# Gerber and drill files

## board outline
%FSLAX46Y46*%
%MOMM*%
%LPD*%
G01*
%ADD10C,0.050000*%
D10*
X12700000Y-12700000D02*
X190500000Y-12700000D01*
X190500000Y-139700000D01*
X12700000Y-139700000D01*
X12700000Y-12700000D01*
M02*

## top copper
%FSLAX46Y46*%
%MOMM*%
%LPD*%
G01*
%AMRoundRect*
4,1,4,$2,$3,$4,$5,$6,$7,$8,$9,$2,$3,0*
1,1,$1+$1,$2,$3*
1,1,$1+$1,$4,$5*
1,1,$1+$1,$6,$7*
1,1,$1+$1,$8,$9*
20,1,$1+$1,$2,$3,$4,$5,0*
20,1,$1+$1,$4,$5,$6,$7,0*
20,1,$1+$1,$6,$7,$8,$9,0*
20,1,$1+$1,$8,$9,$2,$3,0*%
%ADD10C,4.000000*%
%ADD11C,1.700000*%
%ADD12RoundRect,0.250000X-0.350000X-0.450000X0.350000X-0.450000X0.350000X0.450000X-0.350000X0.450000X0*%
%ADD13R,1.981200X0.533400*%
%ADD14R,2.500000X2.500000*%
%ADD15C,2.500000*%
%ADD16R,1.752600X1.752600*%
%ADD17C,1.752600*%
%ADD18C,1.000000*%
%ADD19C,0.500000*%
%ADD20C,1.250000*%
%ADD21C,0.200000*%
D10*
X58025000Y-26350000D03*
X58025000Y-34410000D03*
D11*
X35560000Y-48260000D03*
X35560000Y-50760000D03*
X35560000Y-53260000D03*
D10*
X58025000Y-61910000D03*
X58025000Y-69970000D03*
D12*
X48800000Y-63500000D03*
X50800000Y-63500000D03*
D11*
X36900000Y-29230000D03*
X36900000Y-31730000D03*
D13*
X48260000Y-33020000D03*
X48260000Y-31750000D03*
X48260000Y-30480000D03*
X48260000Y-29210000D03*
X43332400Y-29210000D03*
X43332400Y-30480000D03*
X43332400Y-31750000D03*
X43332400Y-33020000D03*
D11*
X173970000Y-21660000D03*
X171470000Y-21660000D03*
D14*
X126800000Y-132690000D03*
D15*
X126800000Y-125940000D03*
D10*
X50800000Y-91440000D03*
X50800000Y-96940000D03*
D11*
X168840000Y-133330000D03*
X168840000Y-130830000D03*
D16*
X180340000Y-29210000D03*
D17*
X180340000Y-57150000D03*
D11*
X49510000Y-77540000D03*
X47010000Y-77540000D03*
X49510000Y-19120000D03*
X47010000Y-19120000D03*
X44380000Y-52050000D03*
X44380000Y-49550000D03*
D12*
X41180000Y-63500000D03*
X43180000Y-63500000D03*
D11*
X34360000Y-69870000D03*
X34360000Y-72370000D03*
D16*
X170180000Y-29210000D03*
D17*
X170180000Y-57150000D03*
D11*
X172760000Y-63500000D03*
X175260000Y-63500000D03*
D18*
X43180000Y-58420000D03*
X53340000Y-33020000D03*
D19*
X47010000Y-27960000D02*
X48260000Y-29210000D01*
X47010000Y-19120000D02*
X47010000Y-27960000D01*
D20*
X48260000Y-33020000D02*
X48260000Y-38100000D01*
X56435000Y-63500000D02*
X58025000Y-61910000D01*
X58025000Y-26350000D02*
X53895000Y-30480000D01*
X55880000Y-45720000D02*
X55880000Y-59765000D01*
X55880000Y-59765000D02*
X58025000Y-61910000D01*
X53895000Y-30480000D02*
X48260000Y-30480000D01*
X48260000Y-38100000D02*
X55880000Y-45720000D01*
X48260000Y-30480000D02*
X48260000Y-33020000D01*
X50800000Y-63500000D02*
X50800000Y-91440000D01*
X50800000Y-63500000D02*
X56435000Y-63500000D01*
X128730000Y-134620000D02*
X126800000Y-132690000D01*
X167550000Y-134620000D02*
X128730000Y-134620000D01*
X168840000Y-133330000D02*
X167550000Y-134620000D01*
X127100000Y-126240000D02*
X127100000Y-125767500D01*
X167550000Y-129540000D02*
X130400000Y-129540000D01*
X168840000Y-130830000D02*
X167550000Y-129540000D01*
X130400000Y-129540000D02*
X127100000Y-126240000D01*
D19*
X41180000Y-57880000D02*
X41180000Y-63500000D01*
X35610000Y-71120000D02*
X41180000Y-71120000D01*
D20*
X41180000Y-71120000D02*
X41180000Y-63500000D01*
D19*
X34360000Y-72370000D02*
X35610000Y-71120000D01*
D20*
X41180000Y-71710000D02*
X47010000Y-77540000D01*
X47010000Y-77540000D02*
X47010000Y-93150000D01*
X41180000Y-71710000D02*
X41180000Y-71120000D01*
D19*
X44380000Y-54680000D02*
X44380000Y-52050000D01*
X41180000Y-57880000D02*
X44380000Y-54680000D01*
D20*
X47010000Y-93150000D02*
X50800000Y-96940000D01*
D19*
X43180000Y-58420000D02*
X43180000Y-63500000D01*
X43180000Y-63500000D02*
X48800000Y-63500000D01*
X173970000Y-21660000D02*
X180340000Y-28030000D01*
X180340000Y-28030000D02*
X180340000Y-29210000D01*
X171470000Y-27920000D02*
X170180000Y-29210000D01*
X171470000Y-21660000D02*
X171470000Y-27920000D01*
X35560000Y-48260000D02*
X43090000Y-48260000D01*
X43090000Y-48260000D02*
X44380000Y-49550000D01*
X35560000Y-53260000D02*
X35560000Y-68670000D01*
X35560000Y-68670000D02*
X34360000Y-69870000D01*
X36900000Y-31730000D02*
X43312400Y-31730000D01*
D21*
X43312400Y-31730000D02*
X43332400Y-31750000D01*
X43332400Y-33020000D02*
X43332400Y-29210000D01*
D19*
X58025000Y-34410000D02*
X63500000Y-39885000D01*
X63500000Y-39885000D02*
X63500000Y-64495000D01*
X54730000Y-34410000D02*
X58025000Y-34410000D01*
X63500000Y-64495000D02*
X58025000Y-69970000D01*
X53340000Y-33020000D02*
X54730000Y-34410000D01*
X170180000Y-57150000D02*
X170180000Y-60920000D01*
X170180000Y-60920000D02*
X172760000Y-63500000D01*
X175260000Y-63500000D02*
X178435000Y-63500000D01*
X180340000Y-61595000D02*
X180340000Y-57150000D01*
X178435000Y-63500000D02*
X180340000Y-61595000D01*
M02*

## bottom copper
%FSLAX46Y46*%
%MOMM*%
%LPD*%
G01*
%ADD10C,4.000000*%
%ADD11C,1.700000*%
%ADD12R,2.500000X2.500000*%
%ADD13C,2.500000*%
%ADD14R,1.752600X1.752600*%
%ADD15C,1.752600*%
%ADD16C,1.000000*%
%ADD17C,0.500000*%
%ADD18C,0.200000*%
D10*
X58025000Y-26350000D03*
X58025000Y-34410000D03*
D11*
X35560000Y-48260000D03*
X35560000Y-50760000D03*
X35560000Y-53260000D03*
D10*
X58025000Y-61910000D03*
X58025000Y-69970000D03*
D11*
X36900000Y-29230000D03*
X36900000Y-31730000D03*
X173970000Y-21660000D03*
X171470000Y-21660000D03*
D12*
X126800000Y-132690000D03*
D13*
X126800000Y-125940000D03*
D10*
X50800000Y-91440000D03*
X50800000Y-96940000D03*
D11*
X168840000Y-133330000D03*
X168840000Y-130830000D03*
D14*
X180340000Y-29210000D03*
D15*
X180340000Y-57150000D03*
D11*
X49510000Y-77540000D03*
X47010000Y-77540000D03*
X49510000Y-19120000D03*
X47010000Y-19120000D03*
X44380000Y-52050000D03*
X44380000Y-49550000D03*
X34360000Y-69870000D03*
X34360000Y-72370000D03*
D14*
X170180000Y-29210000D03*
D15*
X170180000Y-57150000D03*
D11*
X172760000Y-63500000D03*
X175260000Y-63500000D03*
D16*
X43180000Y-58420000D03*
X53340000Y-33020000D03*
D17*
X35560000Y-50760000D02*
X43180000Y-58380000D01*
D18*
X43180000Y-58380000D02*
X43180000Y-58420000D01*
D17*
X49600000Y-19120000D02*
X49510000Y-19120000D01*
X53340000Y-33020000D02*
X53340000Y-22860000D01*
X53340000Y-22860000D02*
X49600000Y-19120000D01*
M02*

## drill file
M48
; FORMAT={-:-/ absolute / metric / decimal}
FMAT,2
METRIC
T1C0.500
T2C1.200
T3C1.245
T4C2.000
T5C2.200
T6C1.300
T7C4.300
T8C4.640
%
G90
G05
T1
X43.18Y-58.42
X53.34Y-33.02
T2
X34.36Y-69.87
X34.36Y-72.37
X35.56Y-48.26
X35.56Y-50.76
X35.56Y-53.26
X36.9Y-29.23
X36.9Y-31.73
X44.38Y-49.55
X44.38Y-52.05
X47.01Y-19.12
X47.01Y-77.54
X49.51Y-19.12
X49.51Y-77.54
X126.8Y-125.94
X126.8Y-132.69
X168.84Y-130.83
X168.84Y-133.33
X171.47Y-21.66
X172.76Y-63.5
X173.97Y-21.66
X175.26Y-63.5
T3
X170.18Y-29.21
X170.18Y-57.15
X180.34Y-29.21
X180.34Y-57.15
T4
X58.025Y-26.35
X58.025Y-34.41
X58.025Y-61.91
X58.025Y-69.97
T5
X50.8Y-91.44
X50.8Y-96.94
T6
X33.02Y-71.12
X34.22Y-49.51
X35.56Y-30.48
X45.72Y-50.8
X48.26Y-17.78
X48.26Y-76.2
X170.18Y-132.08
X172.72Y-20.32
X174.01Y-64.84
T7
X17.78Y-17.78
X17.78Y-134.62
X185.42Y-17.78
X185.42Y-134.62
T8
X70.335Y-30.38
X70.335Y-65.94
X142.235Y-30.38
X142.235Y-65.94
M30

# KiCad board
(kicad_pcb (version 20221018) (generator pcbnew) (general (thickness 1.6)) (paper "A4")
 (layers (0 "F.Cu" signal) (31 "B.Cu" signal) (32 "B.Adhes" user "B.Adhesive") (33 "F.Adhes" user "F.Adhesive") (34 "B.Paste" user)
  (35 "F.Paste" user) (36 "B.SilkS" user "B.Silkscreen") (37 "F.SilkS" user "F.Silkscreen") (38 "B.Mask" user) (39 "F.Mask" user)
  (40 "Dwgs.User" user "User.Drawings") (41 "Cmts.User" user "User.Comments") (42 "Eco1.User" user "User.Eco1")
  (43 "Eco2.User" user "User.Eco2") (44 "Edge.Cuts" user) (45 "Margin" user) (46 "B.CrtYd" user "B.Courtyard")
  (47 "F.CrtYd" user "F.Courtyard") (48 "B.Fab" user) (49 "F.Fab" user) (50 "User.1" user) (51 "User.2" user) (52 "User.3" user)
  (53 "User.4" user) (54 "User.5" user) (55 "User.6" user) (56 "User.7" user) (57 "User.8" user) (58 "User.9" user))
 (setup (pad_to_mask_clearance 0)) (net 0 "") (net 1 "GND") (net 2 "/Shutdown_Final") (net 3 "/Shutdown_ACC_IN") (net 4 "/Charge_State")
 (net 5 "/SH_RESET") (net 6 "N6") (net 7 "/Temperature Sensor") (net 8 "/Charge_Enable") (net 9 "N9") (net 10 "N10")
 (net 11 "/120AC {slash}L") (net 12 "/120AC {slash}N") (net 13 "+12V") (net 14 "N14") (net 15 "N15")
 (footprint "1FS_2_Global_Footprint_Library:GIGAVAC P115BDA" (layer "F.Cu") (at 146.925 46.95 180)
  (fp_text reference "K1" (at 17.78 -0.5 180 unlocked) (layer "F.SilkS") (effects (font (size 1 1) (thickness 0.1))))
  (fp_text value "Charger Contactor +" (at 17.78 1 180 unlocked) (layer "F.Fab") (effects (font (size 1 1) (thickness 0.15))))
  (pad "" np_thru_hole circle (at 4.69 16.57 180) (size 4.64 4.64) (drill 4.64) (layers "F&B.Cu" "*.Mask"))
  (pad "" np_thru_hole circle (at 76.59 16.57 180) (size 4.64 4.64) (drill 4.64) (layers "F&B.Cu" "*.Mask"))
  (pad "3" thru_hole circle (at 88.9 20.6 180) (size 4 4) (drill 2) (layers "*.Cu" "*.Mask") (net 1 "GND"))
  (pad "4" thru_hole circle (at 88.9 12.54 180) (size 4 4) (drill 2) (layers "*.Cu" "*.Mask") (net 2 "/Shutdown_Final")))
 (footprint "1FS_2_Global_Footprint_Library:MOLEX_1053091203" (layer "F.Cu") (at 35.56 48.26 -90)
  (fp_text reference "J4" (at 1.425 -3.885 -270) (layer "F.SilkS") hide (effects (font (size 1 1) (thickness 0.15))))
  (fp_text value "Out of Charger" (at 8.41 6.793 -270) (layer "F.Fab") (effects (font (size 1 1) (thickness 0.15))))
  (pad "" np_thru_hole circle (at 1.25 1.34 270) (size 1.3 1.3) (drill 1.3) (layers "*.Cu" "*.Mask"))
  (pad "1" thru_hole circle (at 0 0 270) (size 1.7 1.7) (drill 1.2) (layers "*.Cu") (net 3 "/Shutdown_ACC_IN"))
  (pad "2" thru_hole circle (at 2.5 0 270) (size 1.7 1.7) (drill 1.2) (layers "*.Cu") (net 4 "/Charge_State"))
  (pad "3" thru_hole circle (at 5 0 270) (size 1.7 1.7) (drill 1.2) (layers "*.Cu") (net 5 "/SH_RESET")))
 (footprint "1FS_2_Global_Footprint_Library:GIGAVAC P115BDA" (layer "F.Cu") (at 146.925 82.51 180)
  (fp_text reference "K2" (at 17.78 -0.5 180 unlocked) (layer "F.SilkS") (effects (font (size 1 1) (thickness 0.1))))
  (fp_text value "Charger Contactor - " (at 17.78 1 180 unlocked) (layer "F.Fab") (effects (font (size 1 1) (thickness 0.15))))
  (pad "" np_thru_hole circle (at 4.69 16.57 180) (size 4.64 4.64) (drill 4.64) (layers "F&B.Cu" "*.Mask"))
  (pad "" np_thru_hole circle (at 76.59 16.57 180) (size 4.64 4.64) (drill 4.64) (layers "F&B.Cu" "*.Mask"))
  (pad "3" thru_hole circle (at 88.9 20.6 180) (size 4 4) (drill 2) (layers "*.Cu" "*.Mask") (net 1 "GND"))
  (pad "4" thru_hole circle (at 88.9 12.54 180) (size 4 4) (drill 2) (layers "*.Cu" "*.Mask") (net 2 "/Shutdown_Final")))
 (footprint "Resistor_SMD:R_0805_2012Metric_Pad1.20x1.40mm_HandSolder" (layer "F.Cu") (at 49.8 63.5)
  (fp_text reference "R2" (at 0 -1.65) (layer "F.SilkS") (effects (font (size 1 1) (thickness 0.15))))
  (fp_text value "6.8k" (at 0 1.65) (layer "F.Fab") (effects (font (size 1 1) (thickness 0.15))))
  (pad "1" smd roundrect (at -1 0) (size 1.2 1.4) (layers "F.Cu" "F.Paste" "F.Mask") (roundrect_rratio 0.2083333333) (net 4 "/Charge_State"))
  (pad "2" smd roundrect (at 1 0) (size 1.2 1.4) (layers "F.Cu" "F.Paste" "F.Mask") (roundrect_rratio 0.2083333333) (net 1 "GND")))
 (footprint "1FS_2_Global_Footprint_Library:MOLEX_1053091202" (layer "F.Cu") (at 36.9 29.23 -90)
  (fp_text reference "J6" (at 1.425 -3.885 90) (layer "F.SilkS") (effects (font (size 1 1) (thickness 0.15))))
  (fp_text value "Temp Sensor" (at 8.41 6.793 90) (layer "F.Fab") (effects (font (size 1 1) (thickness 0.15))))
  (pad "" np_thru_hole circle (at 1.25 1.34 270) (size 1.3 1.3) (drill 1.3) (layers "*.Cu" "*.Mask"))
  (pad "1" thru_hole circle (at 0 0 270) (size 1.7 1.7) (drill 1.2) (layers "*.Cu") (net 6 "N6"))
  (pad "2" thru_hole circle (at 2.5 0 270) (size 1.7 1.7) (drill 1.2) (layers "*.Cu") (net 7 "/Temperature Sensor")))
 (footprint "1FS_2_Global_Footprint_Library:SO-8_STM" (layer "F.Cu") (at 45.7962 31.115 180)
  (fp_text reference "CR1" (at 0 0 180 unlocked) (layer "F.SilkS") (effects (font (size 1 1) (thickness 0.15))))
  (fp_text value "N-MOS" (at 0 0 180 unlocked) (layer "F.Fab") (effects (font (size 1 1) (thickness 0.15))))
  (pad "1" smd rect (at -2.4638 -1.905 180) (size 1.9812 0.5334) (layers "F.Cu" "F.Paste" "F.Mask") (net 1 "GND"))
  (pad "2" smd rect (at -2.4638 -0.635 180) (size 1.9812 0.5334) (layers "F.Cu" "F.Paste" "F.Mask") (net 1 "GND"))
  (pad "3" smd rect (at -2.4638 0.635 180) (size 1.9812 0.5334) (layers "F.Cu" "F.Paste" "F.Mask") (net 1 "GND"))
  (pad "4" smd rect (at -2.4638 1.905 180) (size 1.9812 0.5334) (layers "F.Cu" "F.Paste" "F.Mask") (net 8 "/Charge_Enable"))
  (pad "5" smd rect (at 2.4638 1.905 180) (size 1.9812 0.5334) (layers "F.Cu" "F.Paste" "F.Mask") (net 7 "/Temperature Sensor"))
  (pad "6" smd rect (at 2.4638 0.635 180) (size 1.9812 0.5334) (layers "F.Cu" "F.Paste" "F.Mask") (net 7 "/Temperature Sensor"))
  (pad "7" smd rect (at 2.4638 -0.635 180) (size 1.9812 0.5334) (layers "F.Cu" "F.Paste" "F.Mask") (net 7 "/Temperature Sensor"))
  (pad "8" smd rect (at 2.4638 -1.905 180) (size 1.9812 0.5334) (layers "F.Cu" "F.Paste" "F.Mask") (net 7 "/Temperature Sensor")))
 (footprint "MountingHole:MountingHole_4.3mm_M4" (layer "F.Cu") (at 185.42 134.62)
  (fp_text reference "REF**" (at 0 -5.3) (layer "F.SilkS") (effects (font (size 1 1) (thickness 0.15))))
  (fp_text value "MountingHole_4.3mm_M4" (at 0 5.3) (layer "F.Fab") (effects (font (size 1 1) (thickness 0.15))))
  (pad "" np_thru_hole circle (at 0 0) (size 4.3 4.3) (drill 4.3) (layers "*.Cu" "*.Mask")))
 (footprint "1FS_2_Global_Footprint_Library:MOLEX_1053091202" (layer "F.Cu") (at 173.97 21.66 180)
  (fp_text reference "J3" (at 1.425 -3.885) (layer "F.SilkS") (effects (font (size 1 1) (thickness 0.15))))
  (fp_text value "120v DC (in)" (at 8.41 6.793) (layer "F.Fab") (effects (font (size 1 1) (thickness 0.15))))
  (pad "" np_thru_hole circle (at 1.25 1.34 180) (size 1.3 1.3) (drill 1.3) (layers "*.Cu" "*.Mask"))
  (pad "1" thru_hole circle (at 0 0 180) (size 1.7 1.7) (drill 1.2) (layers "*.Cu") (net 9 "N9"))
  (pad "2" thru_hole circle (at 2.5 0 180) (size 1.7 1.7) (drill 1.2) (layers "*.Cu") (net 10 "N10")))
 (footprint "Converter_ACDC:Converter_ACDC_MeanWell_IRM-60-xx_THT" (layer "F.Cu") (at 126.8 132.69 180)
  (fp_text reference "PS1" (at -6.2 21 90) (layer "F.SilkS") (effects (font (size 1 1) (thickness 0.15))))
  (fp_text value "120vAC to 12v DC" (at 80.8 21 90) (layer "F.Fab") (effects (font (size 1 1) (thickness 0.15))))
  (pad "1" thru_hole rect (at 0 0 180) (size 2.5 2.5) (drill 1.2) (layers "*.Cu" "*.Mask") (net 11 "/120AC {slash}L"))
  (pad "2" thru_hole circle (at 0 6.75 180) (size 2.5 2.5) (drill 1.2) (layers "*.Cu" "*.Mask") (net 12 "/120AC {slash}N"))
  (pad "3" thru_hole circle (at 76 41.25 180) (size 4 4) (drill 2.2) (layers "*.Cu" "*.Mask") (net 1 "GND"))
  (pad "4" thru_hole circle (at 76 35.75 180) (size 4 4) (drill 2.2) (layers "*.Cu" "*.Mask") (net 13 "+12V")))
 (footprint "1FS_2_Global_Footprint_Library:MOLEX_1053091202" (layer "F.Cu") (at 168.84 133.33 90)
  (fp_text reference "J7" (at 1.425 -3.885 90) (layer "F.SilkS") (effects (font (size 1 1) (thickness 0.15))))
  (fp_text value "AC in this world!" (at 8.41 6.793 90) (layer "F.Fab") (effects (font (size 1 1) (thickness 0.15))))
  (pad "" np_thru_hole circle (at 1.25 1.34 90) (size 1.3 1.3) (drill 1.3) (layers "*.Cu" "*.Mask"))
  (pad "1" thru_hole circle (at 0 0 90) (size 1.7 1.7) (drill 1.2) (layers "*.Cu") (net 11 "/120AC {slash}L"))
  (pad "2" thru_hole circle (at 2.5 0 90) (size 1.7 1.7) (drill 1.2) (layers "*.Cu") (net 12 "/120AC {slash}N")))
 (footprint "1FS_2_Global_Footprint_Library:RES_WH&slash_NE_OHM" (layer "F.Cu") (at 180.34 29.21 -90)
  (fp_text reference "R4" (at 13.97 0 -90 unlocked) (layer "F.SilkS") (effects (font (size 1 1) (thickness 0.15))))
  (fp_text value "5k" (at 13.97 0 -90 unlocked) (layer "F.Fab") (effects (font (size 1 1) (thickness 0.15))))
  (pad "1" thru_hole rect (at 0 0 270) (size 1.7526 1.7526) (drill 1.2446) (layers "*.Cu" "*.Mask") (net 9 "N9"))
  (pad "2" thru_hole circle (at 27.94 0 270) (size 1.7526 1.7526) (drill 1.2446) (layers "*.Cu" "*.Mask") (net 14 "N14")))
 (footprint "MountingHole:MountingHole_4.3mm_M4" (layer "F.Cu") (at 17.78 17.78)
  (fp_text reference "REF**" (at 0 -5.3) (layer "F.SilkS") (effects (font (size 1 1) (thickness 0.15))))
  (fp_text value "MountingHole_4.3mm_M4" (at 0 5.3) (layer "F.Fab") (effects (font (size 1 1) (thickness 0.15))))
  (pad "" np_thru_hole circle (at 0 0) (size 4.3 4.3) (drill 4.3) (layers "F&B.Cu" "*.Mask")))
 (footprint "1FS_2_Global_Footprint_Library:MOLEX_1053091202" (layer "F.Cu") (at 49.51 77.54 180)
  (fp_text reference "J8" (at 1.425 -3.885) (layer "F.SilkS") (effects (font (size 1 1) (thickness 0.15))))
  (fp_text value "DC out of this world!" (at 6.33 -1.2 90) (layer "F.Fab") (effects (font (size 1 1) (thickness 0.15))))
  (pad "" np_thru_hole circle (at 1.25 1.34 180) (size 1.3 1.3) (drill 1.3) (layers "*.Cu" "*.Mask"))
  (pad "1" thru_hole circle (at 0 0 180) (size 1.7 1.7) (drill 1.2) (layers "*.Cu") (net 1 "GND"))
  (pad "2" thru_hole circle (at 2.5 0 180) (size 1.7 1.7) (drill 1.2) (layers "*.Cu") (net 13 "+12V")))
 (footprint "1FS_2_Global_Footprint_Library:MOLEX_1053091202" (layer "F.Cu") (at 49.51 19.12 180)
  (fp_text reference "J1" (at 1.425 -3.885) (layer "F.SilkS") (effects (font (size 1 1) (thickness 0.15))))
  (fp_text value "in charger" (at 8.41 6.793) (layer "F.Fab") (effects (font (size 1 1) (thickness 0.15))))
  (pad "" np_thru_hole circle (at 1.25 1.34 180) (size 1.3 1.3) (drill 1.3) (layers "*.Cu" "*.Mask"))
  (pad "1" thru_hole circle (at 0 0 180) (size 1.7 1.7) (drill 1.2) (layers "*.Cu") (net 2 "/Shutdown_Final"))
  (pad "2" thru_hole circle (at 2.5 0 180) (size 1.7 1.7) (drill 1.2) (layers "*.Cu") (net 8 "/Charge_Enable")))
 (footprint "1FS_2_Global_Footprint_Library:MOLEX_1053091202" (layer "F.Cu") (at 44.38 52.05 90)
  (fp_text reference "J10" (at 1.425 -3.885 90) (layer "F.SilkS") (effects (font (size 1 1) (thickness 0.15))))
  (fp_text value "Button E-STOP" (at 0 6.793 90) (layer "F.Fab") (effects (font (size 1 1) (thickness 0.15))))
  (pad "" np_thru_hole circle (at 1.25 1.34 90) (size 1.3 1.3) (drill 1.3) (layers "*.Cu" "*.Mask"))
  (pad "1" thru_hole circle (at 0 0 90) (size 1.7 1.7) (drill 1.2) (layers "*.Cu") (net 13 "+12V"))
  (pad "2" thru_hole circle (at 2.5 0 90) (size 1.7 1.7) (drill 1.2) (layers "*.Cu") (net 3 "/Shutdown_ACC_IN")))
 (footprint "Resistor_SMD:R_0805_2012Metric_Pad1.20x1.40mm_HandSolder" (layer "F.Cu") (at 42.18 63.5)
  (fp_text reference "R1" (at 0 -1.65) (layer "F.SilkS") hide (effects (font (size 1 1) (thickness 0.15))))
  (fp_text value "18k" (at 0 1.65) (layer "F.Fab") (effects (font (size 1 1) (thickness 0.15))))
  (pad "1" smd roundrect (at -1 0) (size 1.2 1.4) (layers "F.Cu" "F.Paste" "F.Mask") (roundrect_rratio 0.2083333333) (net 13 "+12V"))
  (pad "2" smd roundrect (at 1 0) (size 1.2 1.4) (layers "F.Cu" "F.Paste" "F.Mask") (roundrect_rratio 0.2083333333) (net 4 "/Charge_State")))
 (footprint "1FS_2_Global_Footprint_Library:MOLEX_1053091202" (layer "F.Cu") (at 34.36 69.87 -90)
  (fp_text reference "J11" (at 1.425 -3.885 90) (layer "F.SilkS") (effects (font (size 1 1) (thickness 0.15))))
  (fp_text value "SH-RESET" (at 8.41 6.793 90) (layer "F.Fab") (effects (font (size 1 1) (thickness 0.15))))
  (pad "" np_thru_hole circle (at 1.25 1.34 270) (size 1.3 1.3) (drill 1.3) (layers "*.Cu" "*.Mask"))
  (pad "1" thru_hole circle (at 0 0 270) (size 1.7 1.7) (drill 1.2) (layers "*.Cu") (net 5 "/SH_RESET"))
  (pad "2" thru_hole circle (at 2.5 0 270) (size 1.7 1.7) (drill 1.2) (layers "*.Cu") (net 13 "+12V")))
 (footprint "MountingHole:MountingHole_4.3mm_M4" (layer "F.Cu") (at 185.42 17.78)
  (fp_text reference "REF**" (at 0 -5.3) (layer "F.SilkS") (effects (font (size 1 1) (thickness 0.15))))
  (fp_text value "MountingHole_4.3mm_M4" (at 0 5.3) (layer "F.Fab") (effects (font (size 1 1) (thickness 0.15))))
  (pad "" np_thru_hole circle (at 0 0) (size 4.3 4.3) (drill 4.3) (layers "F&B.Cu" "*.Mask")))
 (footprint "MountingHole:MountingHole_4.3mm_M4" (layer "F.Cu") (at 17.78 134.62)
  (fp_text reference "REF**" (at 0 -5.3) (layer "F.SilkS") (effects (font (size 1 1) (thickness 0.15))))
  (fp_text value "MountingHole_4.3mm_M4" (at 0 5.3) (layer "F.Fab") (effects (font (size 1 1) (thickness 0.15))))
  (pad "" np_thru_hole circle (at 0 0) (size 4.3 4.3) (drill 4.3) (layers "F&B.Cu" "*.Mask")))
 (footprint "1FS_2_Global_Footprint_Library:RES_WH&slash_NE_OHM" (layer "F.Cu") (at 170.18 29.21 -90)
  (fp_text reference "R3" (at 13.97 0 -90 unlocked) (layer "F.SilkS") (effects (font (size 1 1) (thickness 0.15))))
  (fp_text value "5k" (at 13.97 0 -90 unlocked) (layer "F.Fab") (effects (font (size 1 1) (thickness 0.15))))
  (pad "1" thru_hole rect (at 0 0 270) (size 1.7526 1.7526) (drill 1.2446) (layers "*.Cu" "*.Mask") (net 10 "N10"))
  (pad "2" thru_hole circle (at 27.94 0 270) (size 1.7526 1.7526) (drill 1.2446) (layers "*.Cu" "*.Mask") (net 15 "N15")))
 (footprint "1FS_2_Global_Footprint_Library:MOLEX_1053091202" (layer "F.Cu") (at 172.76 63.5)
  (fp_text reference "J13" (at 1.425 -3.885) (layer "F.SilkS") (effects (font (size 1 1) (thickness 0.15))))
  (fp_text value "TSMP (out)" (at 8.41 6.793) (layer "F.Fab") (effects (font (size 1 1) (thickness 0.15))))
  (pad "" np_thru_hole circle (at 1.25 1.34) (size 1.3 1.3) (drill 1.3) (layers "*.Cu" "*.Mask"))
  (pad "1" thru_hole circle (at 0 0) (size 1.7 1.7) (drill 1.2) (layers "*.Cu") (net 15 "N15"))
  (pad "2" thru_hole circle (at 2.5 0) (size 1.7 1.7) (drill 1.2) (layers "*.Cu") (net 14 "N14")))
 (gr_rect (start 12.7 12.7) (end 190.5 139.7) (stroke (width 0.05) (type default)) (fill none) (layer "Edge.Cuts"))
 (segment (start 47.01 27.96) (end 48.26 29.21) (width 0.5) (layer "F.Cu") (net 8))
 (segment (start 47.01 19.12) (end 47.01 27.96) (width 0.5) (layer "F.Cu") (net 8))
 (segment (start 48.26 33.02) (end 48.26 38.1) (width 1.25) (layer "F.Cu") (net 1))
 (segment (start 56.435 63.5) (end 58.025 61.91) (width 1.25) (layer "F.Cu") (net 1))
 (segment (start 58.025 26.35) (end 53.895 30.48) (width 1.25) (layer "F.Cu") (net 1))
 (segment (start 55.88 45.72) (end 55.88 59.765) (width 1.25) (layer "F.Cu") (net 1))
 (segment (start 55.88 59.765) (end 58.025 61.91) (width 1.25) (layer "F.Cu") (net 1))
 (segment (start 53.895 30.48) (end 48.26 30.48) (width 1.25) (layer "F.Cu") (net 1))
 (segment (start 48.26 38.1) (end 55.88 45.72) (width 1.25) (layer "F.Cu") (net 1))
 (segment (start 48.26 30.48) (end 48.26 33.02) (width 1.25) (layer "F.Cu") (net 1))
 (segment (start 50.8 63.5) (end 50.8 91.44) (width 1.25) (layer "F.Cu") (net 1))
 (segment (start 50.8 63.5) (end 56.435 63.5) (width 1.25) (layer "F.Cu") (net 1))
 (segment (start 128.73 134.62) (end 126.8 132.69) (width 1.25) (layer "F.Cu") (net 11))
 (segment (start 167.55 134.62) (end 128.73 134.62) (width 1.25) (layer "F.Cu") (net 11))
 (segment (start 168.84 133.33) (end 167.55 134.62) (width 1.25) (layer "F.Cu") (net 11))
 (segment (start 127.1 126.24) (end 127.1 125.7675) (width 1.25) (layer "F.Cu") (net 12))
 (segment (start 167.55 129.54) (end 130.4 129.54) (width 1.25) (layer "F.Cu") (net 12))
 (segment (start 168.84 130.83) (end 167.55 129.54) (width 1.25) (layer "F.Cu") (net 12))
 (segment (start 130.4 129.54) (end 127.1 126.24) (width 1.25) (layer "F.Cu") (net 12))
 (segment (start 41.18 57.88) (end 41.18 63.5) (width 0.5) (layer "F.Cu") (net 13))
 (segment (start 35.61 71.12) (end 41.18 71.12) (width 0.5) (layer "F.Cu") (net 13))
 (segment (start 41.18 71.12) (end 41.18 63.5) (width 1.25) (layer "F.Cu") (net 13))
 (segment (start 34.36 72.37) (end 35.61 71.12) (width 0.5) (layer "F.Cu") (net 13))
 (segment (start 41.18 71.71) (end 47.01 77.54) (width 1.25) (layer "F.Cu") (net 13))
 (segment (start 47.01 77.54) (end 47.01 93.15) (width 1.25) (layer "F.Cu") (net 13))
 (segment (start 41.18 71.71) (end 41.18 71.12) (width 1.25) (layer "F.Cu") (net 13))
 (segment (start 44.38 54.68) (end 44.38 52.05) (width 0.5) (layer "F.Cu") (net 13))
 (segment (start 41.18 57.88) (end 44.38 54.68) (width 0.5) (layer "F.Cu") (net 13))
 (segment (start 47.01 93.15) (end 50.8 96.94) (width 1.25) (layer "F.Cu") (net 13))
 (segment (start 43.18 58.42) (end 43.18 63.5) (width 0.5) (layer "F.Cu") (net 4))
 (segment (start 43.18 63.5) (end 48.8 63.5) (width 0.5) (layer "F.Cu") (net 4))
 (via (at 43.18 58.42) (size 1) (drill 0.5) (layers "F.Cu" "B.Cu") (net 4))
 (segment (start 35.56 50.76) (end 43.18 58.38) (width 0.5) (layer "B.Cu") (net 4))
 (segment (start 43.18 58.38) (end 43.18 58.42) (width 0.2) (layer "B.Cu") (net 4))
 (segment (start 173.97 21.66) (end 180.34 28.03) (width 0.5) (layer "F.Cu") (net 9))
 (segment (start 180.34 28.03) (end 180.34 29.21) (width 0.5) (layer "F.Cu") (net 9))
 (segment (start 171.47 27.92) (end 170.18 29.21) (width 0.5) (layer "F.Cu") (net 10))
 (segment (start 171.47 21.66) (end 171.47 27.92) (width 0.5) (layer "F.Cu") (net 10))
 (segment (start 35.56 48.26) (end 43.09 48.26) (width 0.5) (layer "F.Cu") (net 3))
 (segment (start 43.09 48.26) (end 44.38 49.55) (width 0.5) (layer "F.Cu") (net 3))
 (segment (start 35.56 53.26) (end 35.56 68.67) (width 0.5) (layer "F.Cu") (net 5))
 (segment (start 35.56 68.67) (end 34.36 69.87) (width 0.5) (layer "F.Cu") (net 5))
 (segment (start 36.9 31.73) (end 43.3124 31.73) (width 0.5) (layer "F.Cu") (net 7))
 (segment (start 43.3124 31.73) (end 43.3324 31.75) (width 0.2) (layer "F.Cu") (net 7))
 (segment (start 43.3324 33.02) (end 43.3324 29.21) (width 0.2) (layer "F.Cu") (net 7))
 (segment (start 58.025 34.41) (end 63.5 39.885) (width 0.5) (layer "F.Cu") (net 2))
 (segment (start 63.5 39.885) (end 63.5 64.495) (width 0.5) (layer "F.Cu") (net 2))
 (segment (start 54.73 34.41) (end 58.025 34.41) (width 0.5) (layer "F.Cu") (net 2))
 (segment (start 63.5 64.495) (end 58.025 69.97) (width 0.5) (layer "F.Cu") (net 2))
 (segment (start 53.34 33.02) (end 54.73 34.41) (width 0.5) (layer "F.Cu") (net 2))
 (via (at 53.34 33.02) (size 1) (drill 0.5) (layers "F.Cu" "B.Cu") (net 2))
 (segment (start 49.6 19.12) (end 49.51 19.12) (width 0.5) (layer "B.Cu") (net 2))
 (segment (start 53.34 33.02) (end 53.34 22.86) (width 0.5) (layer "B.Cu") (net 2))
 (segment (start 53.34 22.86) (end 49.6 19.12) (width 0.5) (layer "B.Cu") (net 2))
 (segment (start 170.18 57.15) (end 170.18 60.92) (width 0.5) (layer "F.Cu") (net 15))
 (segment (start 170.18 60.92) (end 172.76 63.5) (width 0.5) (layer "F.Cu") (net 15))
 (segment (start 175.26 63.5) (end 178.435 63.5) (width 0.5) (layer "F.Cu") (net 14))
 (segment (start 180.34 61.595) (end 180.34 57.15) (width 0.5) (layer "F.Cu") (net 14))
 (segment (start 178.435 63.5) (end 180.34 61.595) (width 0.5) (layer "F.Cu") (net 14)))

